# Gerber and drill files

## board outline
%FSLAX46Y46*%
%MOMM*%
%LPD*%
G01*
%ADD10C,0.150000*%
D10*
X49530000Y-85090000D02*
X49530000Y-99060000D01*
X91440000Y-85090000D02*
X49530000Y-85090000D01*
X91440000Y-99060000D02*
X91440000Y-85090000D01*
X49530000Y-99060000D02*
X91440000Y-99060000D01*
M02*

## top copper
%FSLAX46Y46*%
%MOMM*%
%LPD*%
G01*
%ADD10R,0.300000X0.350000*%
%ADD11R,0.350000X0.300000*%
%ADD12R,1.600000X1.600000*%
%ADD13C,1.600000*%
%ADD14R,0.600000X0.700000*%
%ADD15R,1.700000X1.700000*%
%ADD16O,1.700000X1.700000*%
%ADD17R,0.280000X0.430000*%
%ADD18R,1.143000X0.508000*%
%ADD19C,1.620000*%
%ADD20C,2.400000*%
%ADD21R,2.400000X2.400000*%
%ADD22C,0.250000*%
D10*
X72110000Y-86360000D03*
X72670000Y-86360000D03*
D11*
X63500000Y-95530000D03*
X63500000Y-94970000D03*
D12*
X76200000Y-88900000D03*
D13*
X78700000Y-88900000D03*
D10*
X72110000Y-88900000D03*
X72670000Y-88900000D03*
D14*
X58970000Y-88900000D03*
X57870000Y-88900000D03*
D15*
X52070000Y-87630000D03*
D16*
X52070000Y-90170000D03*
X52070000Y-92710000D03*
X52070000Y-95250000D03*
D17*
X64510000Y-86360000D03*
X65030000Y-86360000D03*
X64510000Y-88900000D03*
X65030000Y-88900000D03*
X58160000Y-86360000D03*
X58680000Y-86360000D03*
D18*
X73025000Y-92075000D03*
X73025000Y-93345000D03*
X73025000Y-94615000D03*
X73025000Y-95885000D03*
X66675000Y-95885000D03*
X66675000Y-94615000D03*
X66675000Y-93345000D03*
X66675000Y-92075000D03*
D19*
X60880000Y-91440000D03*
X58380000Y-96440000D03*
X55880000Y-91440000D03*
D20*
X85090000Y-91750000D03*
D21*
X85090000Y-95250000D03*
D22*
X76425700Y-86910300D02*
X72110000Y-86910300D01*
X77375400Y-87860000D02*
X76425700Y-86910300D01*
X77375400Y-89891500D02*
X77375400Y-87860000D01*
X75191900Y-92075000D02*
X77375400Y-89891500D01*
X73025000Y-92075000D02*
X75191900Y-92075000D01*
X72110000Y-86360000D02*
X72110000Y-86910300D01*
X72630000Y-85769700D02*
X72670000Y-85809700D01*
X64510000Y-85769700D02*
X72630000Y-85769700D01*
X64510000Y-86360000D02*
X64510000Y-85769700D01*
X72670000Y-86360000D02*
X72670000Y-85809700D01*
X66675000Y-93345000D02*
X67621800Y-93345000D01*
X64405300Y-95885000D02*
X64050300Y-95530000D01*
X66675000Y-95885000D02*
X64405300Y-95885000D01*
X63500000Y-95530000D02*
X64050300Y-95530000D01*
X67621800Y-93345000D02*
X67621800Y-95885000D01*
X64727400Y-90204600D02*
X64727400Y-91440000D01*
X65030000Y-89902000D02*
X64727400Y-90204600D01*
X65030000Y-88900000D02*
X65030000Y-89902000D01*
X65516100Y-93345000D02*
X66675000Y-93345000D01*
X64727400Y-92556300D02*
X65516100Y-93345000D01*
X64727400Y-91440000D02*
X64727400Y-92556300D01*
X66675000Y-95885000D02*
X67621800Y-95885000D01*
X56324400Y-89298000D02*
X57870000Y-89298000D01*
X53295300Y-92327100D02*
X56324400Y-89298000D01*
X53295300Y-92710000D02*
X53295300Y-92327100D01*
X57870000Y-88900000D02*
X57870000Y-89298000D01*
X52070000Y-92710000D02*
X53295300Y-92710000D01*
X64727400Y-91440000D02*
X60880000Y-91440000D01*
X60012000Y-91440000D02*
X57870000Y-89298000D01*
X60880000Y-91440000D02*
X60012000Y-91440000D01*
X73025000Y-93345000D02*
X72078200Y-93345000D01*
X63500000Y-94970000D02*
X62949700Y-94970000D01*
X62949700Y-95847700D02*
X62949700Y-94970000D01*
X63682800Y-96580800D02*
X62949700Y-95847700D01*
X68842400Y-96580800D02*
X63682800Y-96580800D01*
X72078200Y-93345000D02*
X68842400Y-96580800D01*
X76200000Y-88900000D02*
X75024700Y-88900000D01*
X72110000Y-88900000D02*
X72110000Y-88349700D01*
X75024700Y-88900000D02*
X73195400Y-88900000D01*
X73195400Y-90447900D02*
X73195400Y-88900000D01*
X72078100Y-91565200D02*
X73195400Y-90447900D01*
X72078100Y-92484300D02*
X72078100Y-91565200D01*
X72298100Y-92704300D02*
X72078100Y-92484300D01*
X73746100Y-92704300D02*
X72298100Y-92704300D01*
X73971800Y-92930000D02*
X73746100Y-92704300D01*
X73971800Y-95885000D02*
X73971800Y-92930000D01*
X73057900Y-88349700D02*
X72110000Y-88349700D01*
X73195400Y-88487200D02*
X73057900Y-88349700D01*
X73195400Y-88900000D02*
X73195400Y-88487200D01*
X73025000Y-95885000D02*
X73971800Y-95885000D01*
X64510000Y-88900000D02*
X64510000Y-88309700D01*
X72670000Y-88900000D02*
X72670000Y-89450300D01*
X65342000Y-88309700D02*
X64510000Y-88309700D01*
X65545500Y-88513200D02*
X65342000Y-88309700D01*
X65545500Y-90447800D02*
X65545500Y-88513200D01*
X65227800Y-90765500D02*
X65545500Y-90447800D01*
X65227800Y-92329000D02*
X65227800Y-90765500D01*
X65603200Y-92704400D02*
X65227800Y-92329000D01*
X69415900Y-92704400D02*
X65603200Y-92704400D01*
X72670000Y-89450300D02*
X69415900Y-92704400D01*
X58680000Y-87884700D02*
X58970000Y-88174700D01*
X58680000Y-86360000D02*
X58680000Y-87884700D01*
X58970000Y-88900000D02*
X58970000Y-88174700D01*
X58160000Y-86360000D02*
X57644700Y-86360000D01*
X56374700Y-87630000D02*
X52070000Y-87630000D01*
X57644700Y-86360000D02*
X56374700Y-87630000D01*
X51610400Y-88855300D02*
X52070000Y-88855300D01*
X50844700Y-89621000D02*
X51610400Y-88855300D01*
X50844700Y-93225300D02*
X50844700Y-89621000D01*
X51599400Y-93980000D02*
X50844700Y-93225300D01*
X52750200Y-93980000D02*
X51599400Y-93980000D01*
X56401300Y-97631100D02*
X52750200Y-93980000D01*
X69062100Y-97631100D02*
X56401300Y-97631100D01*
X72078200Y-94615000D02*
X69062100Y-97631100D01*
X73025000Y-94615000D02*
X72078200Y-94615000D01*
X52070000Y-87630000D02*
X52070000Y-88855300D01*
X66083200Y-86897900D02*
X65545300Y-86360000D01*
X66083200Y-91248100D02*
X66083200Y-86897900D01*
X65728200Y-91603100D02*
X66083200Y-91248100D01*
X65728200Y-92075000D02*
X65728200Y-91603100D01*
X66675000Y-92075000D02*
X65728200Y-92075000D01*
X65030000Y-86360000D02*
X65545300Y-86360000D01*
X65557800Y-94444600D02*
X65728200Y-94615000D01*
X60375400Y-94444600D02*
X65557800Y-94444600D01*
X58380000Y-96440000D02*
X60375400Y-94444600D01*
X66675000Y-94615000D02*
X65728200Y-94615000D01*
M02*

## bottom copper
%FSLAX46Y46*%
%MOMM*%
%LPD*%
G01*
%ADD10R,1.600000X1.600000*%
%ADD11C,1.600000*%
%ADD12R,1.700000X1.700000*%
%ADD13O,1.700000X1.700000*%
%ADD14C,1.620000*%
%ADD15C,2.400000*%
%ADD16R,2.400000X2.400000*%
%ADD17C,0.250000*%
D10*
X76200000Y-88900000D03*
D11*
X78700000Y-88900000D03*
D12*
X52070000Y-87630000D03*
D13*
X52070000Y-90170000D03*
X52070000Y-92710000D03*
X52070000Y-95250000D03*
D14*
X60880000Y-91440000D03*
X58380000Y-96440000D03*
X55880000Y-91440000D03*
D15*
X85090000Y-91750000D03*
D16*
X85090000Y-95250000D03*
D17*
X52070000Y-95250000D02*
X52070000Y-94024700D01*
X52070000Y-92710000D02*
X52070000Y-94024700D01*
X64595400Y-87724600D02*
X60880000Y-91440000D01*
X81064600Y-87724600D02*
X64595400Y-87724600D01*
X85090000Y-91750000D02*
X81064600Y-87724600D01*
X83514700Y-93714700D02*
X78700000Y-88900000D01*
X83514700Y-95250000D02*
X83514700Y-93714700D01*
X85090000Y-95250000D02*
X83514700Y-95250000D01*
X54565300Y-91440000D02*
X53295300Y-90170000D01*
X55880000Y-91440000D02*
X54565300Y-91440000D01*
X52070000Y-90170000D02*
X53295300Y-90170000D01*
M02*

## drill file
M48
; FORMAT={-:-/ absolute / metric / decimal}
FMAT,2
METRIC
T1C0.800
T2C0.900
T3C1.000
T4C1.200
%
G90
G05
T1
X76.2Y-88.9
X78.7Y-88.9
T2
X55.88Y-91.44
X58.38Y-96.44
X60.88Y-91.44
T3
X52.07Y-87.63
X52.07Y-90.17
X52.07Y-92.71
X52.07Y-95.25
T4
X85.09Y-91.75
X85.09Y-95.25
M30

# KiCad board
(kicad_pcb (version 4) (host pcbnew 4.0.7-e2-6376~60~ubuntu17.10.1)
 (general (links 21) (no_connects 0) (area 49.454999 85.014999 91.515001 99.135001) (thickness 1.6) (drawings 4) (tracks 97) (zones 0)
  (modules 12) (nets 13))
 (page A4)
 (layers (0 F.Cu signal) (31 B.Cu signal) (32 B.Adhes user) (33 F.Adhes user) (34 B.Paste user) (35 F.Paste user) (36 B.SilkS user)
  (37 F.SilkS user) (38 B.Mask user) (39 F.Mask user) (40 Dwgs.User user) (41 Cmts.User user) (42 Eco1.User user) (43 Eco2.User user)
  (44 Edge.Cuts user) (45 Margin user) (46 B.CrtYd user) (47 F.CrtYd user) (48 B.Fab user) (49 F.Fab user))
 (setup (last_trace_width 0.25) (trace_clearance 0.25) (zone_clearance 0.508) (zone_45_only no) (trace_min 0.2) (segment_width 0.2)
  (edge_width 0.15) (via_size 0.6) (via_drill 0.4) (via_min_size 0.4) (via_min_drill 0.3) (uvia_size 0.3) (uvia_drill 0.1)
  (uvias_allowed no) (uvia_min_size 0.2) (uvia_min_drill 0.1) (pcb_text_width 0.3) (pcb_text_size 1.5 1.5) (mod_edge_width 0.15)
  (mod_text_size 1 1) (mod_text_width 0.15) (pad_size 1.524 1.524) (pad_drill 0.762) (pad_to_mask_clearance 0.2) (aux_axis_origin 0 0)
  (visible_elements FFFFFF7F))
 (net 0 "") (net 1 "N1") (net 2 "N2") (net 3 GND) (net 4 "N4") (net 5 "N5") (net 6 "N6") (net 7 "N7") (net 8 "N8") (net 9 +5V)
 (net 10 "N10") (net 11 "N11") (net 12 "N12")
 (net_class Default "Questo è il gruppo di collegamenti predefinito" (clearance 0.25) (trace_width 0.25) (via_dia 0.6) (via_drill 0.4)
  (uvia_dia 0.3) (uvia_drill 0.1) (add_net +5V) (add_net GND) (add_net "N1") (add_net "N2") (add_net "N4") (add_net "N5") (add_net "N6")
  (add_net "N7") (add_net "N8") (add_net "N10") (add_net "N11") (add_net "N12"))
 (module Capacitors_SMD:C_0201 (layer F.Cu) (at 72.39 86.36)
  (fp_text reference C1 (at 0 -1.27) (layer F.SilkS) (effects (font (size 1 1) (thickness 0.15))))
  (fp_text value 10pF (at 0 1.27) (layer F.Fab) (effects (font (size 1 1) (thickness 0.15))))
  (pad 1 smd rect (at -0.28 0) (size 0.3 0.35) (layers F.Cu F.Paste F.Mask) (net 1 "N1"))
  (pad 2 smd rect (at 0.28 0) (size 0.3 0.35) (layers F.Cu F.Paste F.Mask) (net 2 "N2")))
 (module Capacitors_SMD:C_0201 (layer F.Cu) (at 63.5 95.25 90)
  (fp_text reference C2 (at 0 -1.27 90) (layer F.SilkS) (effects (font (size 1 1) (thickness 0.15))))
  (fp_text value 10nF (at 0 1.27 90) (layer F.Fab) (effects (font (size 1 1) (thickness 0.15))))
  (pad 1 smd rect (at -0.28 0 90) (size 0.3 0.35) (layers F.Cu F.Paste F.Mask) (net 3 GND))
  (pad 2 smd rect (at 0.28 0 90) (size 0.3 0.35) (layers F.Cu F.Paste F.Mask) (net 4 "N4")))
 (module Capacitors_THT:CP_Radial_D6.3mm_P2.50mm (layer F.Cu) (at 76.2 88.9)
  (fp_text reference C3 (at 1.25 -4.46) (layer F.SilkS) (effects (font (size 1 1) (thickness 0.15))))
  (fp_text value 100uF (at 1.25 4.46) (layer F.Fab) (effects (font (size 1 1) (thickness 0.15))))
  (pad 1 thru_hole rect (at 0 0) (size 1.6 1.6) (drill 0.8) (layers *.Cu *.Mask) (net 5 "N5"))
  (pad 2 thru_hole circle (at 2.5 0) (size 1.6 1.6) (drill 0.8) (layers *.Cu *.Mask) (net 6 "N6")))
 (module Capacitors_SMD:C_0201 (layer F.Cu) (at 72.39 88.9)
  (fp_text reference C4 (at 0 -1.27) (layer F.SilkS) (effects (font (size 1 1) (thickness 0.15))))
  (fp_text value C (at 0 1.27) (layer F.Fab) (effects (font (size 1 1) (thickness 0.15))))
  (pad 1 smd rect (at -0.28 0) (size 0.3 0.35) (layers F.Cu F.Paste F.Mask) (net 5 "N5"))
  (pad 2 smd rect (at 0.28 0) (size 0.3 0.35) (layers F.Cu F.Paste F.Mask) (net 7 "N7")))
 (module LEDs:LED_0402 (layer F.Cu) (at 58.42 88.9)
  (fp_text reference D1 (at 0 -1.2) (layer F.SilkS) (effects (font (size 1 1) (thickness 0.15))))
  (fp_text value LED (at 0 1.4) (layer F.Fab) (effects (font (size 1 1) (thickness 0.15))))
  (pad 2 smd rect (at 0.55 0 180) (size 0.6 0.7) (layers F.Cu F.Paste F.Mask) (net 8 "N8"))
  (pad 1 smd rect (at -0.55 0 180) (size 0.6 0.7) (layers F.Cu F.Paste F.Mask) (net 3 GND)))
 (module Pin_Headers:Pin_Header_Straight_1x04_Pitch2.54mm (layer F.Cu) (at 52.07 87.63)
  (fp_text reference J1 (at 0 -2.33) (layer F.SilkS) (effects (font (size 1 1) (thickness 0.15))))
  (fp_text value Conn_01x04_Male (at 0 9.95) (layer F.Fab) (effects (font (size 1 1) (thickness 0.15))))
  (pad 1 thru_hole rect (at 0 0) (size 1.7 1.7) (drill 1) (layers *.Cu *.Mask) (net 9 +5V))
  (pad 2 thru_hole oval (at 0 2.54) (size 1.7 1.7) (drill 1) (layers *.Cu *.Mask) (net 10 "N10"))
  (pad 3 thru_hole oval (at 0 5.08) (size 1.7 1.7) (drill 1) (layers *.Cu *.Mask) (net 3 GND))
  (pad 4 thru_hole oval (at 0 7.62) (size 1.7 1.7) (drill 1) (layers *.Cu *.Mask) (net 3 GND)))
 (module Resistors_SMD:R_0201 (layer F.Cu) (at 64.77 86.36)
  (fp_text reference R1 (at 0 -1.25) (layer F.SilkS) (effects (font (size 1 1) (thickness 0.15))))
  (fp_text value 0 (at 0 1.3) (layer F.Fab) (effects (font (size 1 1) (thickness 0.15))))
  (pad 1 smd rect (at -0.26 0) (size 0.28 0.43) (layers F.Cu F.Paste F.Mask) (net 2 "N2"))
  (pad 2 smd rect (at 0.26 0) (size 0.28 0.43) (layers F.Cu F.Paste F.Mask) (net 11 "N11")))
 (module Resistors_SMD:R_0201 (layer F.Cu) (at 64.77 88.9)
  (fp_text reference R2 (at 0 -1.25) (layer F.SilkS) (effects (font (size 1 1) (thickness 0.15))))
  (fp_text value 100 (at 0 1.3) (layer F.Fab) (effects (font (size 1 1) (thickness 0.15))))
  (pad 1 smd rect (at -0.26 0) (size 0.28 0.43) (layers F.Cu F.Paste F.Mask) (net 7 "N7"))
  (pad 2 smd rect (at 0.26 0) (size 0.28 0.43) (layers F.Cu F.Paste F.Mask) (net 3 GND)))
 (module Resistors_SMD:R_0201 (layer F.Cu) (at 58.42 86.36)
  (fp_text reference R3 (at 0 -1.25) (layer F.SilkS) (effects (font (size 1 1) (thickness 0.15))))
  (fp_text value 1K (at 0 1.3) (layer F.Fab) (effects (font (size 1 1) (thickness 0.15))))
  (pad 1 smd rect (at -0.26 0) (size 0.28 0.43) (layers F.Cu F.Paste F.Mask) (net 9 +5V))
  (pad 2 smd rect (at 0.26 0) (size 0.28 0.43) (layers F.Cu F.Paste F.Mask) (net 8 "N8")))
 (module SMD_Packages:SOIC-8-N (layer F.Cu) (at 69.85 93.98 270)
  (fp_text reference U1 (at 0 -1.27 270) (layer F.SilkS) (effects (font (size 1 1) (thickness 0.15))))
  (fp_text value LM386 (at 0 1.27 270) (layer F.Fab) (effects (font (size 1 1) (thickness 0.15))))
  (pad 8 smd rect (at -1.905 -3.175 270) (size 0.508 1.143) (layers F.Cu F.Paste F.Mask) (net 1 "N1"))
  (pad 7 smd rect (at -0.635 -3.175 270) (size 0.508 1.143) (layers F.Cu F.Paste F.Mask) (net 4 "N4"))
  (pad 6 smd rect (at 0.635 -3.175 270) (size 0.508 1.143) (layers F.Cu F.Paste F.Mask) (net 9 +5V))
  (pad 5 smd rect (at 1.905 -3.175 270) (size 0.508 1.143) (layers F.Cu F.Paste F.Mask) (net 5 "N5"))
  (pad 4 smd rect (at 1.905 3.175 270) (size 0.508 1.143) (layers F.Cu F.Paste F.Mask) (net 3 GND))
  (pad 3 smd rect (at 0.635 3.175 270) (size 0.508 1.143) (layers F.Cu F.Paste F.Mask) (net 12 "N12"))
  (pad 2 smd rect (at -0.635 3.175 270) (size 0.508 1.143) (layers F.Cu F.Paste F.Mask) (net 3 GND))
  (pad 1 smd rect (at -1.905 3.175 270) (size 0.508 1.143) (layers F.Cu F.Paste F.Mask) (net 11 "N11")))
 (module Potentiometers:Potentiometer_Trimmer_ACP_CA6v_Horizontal (layer F.Cu) (at 55.88 91.44 270)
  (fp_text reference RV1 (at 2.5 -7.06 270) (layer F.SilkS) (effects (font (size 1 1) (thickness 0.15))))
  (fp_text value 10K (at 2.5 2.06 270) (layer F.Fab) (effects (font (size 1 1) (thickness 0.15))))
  (pad 3 thru_hole circle (at 0 -5 270) (size 1.62 1.62) (drill 0.9) (layers *.Cu *.Mask) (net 3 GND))
  (pad 2 thru_hole circle (at 5 -2.5 270) (size 1.62 1.62) (drill 0.9) (layers *.Cu *.Mask) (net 12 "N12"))
  (pad 1 thru_hole circle (at 0 0 270) (size 1.62 1.62) (drill 0.9) (layers *.Cu *.Mask) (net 10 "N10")))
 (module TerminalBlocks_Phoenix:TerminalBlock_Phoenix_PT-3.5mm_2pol (layer F.Cu) (at 85.09 95.25 90)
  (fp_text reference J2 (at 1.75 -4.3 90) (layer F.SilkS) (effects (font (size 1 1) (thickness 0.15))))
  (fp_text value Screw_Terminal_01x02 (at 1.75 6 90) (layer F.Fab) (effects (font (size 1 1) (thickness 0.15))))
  (pad 2 thru_hole circle (at 3.5 0 90) (size 2.4 2.4) (drill 1.2) (layers *.Cu *.Mask) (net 3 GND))
  (pad 1 thru_hole rect (at 0 0 90) (size 2.4 2.4) (drill 1.2) (layers *.Cu *.Mask) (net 6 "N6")))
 (gr_line (start 49.53 85.09) (end 49.53 99.06) (angle 90) (layer Edge.Cuts) (width 0.15))
 (gr_line (start 91.44 85.09) (end 49.53 85.09) (angle 90) (layer Edge.Cuts) (width 0.15))
 (gr_line (start 91.44 99.06) (end 91.44 85.09) (angle 90) (layer Edge.Cuts) (width 0.15))
 (gr_line (start 49.53 99.06) (end 91.44 99.06) (angle 90) (layer Edge.Cuts) (width 0.15))
 (segment (start 76.4257 86.9103) (end 72.11 86.9103) (width 0.25) (layer F.Cu) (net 1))
 (segment (start 77.3754 87.86) (end 76.4257 86.9103) (width 0.25) (layer F.Cu) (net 1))
 (segment (start 77.3754 89.8915) (end 77.3754 87.86) (width 0.25) (layer F.Cu) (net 1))
 (segment (start 75.1919 92.075) (end 77.3754 89.8915) (width 0.25) (layer F.Cu) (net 1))
 (segment (start 73.025 92.075) (end 75.1919 92.075) (width 0.25) (layer F.Cu) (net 1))
 (segment (start 72.11 86.36) (end 72.11 86.9103) (width 0.25) (layer F.Cu) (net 1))
 (segment (start 72.63 85.7697) (end 72.67 85.8097) (width 0.25) (layer F.Cu) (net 2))
 (segment (start 64.51 85.7697) (end 72.63 85.7697) (width 0.25) (layer F.Cu) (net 2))
 (segment (start 64.51 86.36) (end 64.51 85.7697) (width 0.25) (layer F.Cu) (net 2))
 (segment (start 72.67 86.36) (end 72.67 85.8097) (width 0.25) (layer F.Cu) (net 2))
 (segment (start 66.675 93.345) (end 67.6218 93.345) (width 0.25) (layer F.Cu) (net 3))
 (segment (start 64.4053 95.885) (end 64.0503 95.53) (width 0.25) (layer F.Cu) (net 3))
 (segment (start 66.675 95.885) (end 64.4053 95.885) (width 0.25) (layer F.Cu) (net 3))
 (segment (start 63.5 95.53) (end 64.0503 95.53) (width 0.25) (layer F.Cu) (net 3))
 (segment (start 67.6218 93.345) (end 67.6218 95.885) (width 0.25) (layer F.Cu) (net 3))
 (segment (start 52.07 95.25) (end 52.07 94.0247) (width 0.25) (layer B.Cu) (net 3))
 (segment (start 52.07 92.71) (end 52.07 94.0247) (width 0.25) (layer B.Cu) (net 3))
 (segment (start 64.7274 90.2046) (end 64.7274 91.44) (width 0.25) (layer F.Cu) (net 3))
 (segment (start 65.03 89.902) (end 64.7274 90.2046) (width 0.25) (layer F.Cu) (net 3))
 (segment (start 65.03 88.9) (end 65.03 89.902) (width 0.25) (layer F.Cu) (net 3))
 (segment (start 65.5161 93.345) (end 66.675 93.345) (width 0.25) (layer F.Cu) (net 3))
 (segment (start 64.7274 92.5563) (end 65.5161 93.345) (width 0.25) (layer F.Cu) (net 3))
 (segment (start 64.7274 91.44) (end 64.7274 92.5563) (width 0.25) (layer F.Cu) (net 3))
 (segment (start 66.675 95.885) (end 67.6218 95.885) (width 0.25) (layer F.Cu) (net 3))
 (segment (start 56.3244 89.298) (end 57.87 89.298) (width 0.25) (layer F.Cu) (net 3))
 (segment (start 53.2953 92.3271) (end 56.3244 89.298) (width 0.25) (layer F.Cu) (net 3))
 (segment (start 53.2953 92.71) (end 53.2953 92.3271) (width 0.25) (layer F.Cu) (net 3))
 (segment (start 57.87 88.9) (end 57.87 89.298) (width 0.25) (layer F.Cu) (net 3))
 (segment (start 52.07 92.71) (end 53.2953 92.71) (width 0.25) (layer F.Cu) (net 3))
 (segment (start 64.7274 91.44) (end 60.88 91.44) (width 0.25) (layer F.Cu) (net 3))
 (segment (start 60.012 91.44) (end 57.87 89.298) (width 0.25) (layer F.Cu) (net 3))
 (segment (start 60.88 91.44) (end 60.012 91.44) (width 0.25) (layer F.Cu) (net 3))
 (segment (start 64.5954 87.7246) (end 60.88 91.44) (width 0.25) (layer B.Cu) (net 3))
 (segment (start 81.0646 87.7246) (end 64.5954 87.7246) (width 0.25) (layer B.Cu) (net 3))
 (segment (start 85.09 91.75) (end 81.0646 87.7246) (width 0.25) (layer B.Cu) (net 3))
 (segment (start 73.025 93.345) (end 72.0782 93.345) (width 0.25) (layer F.Cu) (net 4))
 (segment (start 63.5 94.97) (end 62.9497 94.97) (width 0.25) (layer F.Cu) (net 4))
 (segment (start 62.9497 95.8477) (end 62.9497 94.97) (width 0.25) (layer F.Cu) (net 4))
 (segment (start 63.6828 96.5808) (end 62.9497 95.8477) (width 0.25) (layer F.Cu) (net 4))
 (segment (start 68.8424 96.5808) (end 63.6828 96.5808) (width 0.25) (layer F.Cu) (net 4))
 (segment (start 72.0782 93.345) (end 68.8424 96.5808) (width 0.25) (layer F.Cu) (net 4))
 (segment (start 76.2 88.9) (end 75.0247 88.9) (width 0.25) (layer F.Cu) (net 5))
 (segment (start 72.11 88.9) (end 72.11 88.3497) (width 0.25) (layer F.Cu) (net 5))
 (segment (start 75.0247 88.9) (end 73.1954 88.9) (width 0.25) (layer F.Cu) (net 5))
 (segment (start 73.1954 90.4479) (end 73.1954 88.9) (width 0.25) (layer F.Cu) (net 5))
 (segment (start 72.0781 91.5652) (end 73.1954 90.4479) (width 0.25) (layer F.Cu) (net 5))
 (segment (start 72.0781 92.4843) (end 72.0781 91.5652) (width 0.25) (layer F.Cu) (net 5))
 (segment (start 72.2981 92.7043) (end 72.0781 92.4843) (width 0.25) (layer F.Cu) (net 5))
 (segment (start 73.7461 92.7043) (end 72.2981 92.7043) (width 0.25) (layer F.Cu) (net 5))
 (segment (start 73.9718 92.93) (end 73.7461 92.7043) (width 0.25) (layer F.Cu) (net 5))
 (segment (start 73.9718 95.885) (end 73.9718 92.93) (width 0.25) (layer F.Cu) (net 5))
 (segment (start 73.0579 88.3497) (end 72.11 88.3497) (width 0.25) (layer F.Cu) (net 5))
 (segment (start 73.1954 88.4872) (end 73.0579 88.3497) (width 0.25) (layer F.Cu) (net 5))
 (segment (start 73.1954 88.9) (end 73.1954 88.4872) (width 0.25) (layer F.Cu) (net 5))
 (segment (start 73.025 95.885) (end 73.9718 95.885) (width 0.25) (layer F.Cu) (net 5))
 (segment (start 83.5147 93.7147) (end 78.7 88.9) (width 0.25) (layer B.Cu) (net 6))
 (segment (start 83.5147 95.25) (end 83.5147 93.7147) (width 0.25) (layer B.Cu) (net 6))
 (segment (start 85.09 95.25) (end 83.5147 95.25) (width 0.25) (layer B.Cu) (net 6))
 (segment (start 64.51 88.9) (end 64.51 88.3097) (width 0.25) (layer F.Cu) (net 7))
 (segment (start 72.67 88.9) (end 72.67 89.4503) (width 0.25) (layer F.Cu) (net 7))
 (segment (start 65.342 88.3097) (end 64.51 88.3097) (width 0.25) (layer F.Cu) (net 7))
 (segment (start 65.5455 88.5132) (end 65.342 88.3097) (width 0.25) (layer F.Cu) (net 7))
 (segment (start 65.5455 90.4478) (end 65.5455 88.5132) (width 0.25) (layer F.Cu) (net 7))
 (segment (start 65.2278 90.7655) (end 65.5455 90.4478) (width 0.25) (layer F.Cu) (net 7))
 (segment (start 65.2278 92.329) (end 65.2278 90.7655) (width 0.25) (layer F.Cu) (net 7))
 (segment (start 65.6032 92.7044) (end 65.2278 92.329) (width 0.25) (layer F.Cu) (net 7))
 (segment (start 69.4159 92.7044) (end 65.6032 92.7044) (width 0.25) (layer F.Cu) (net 7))
 (segment (start 72.67 89.4503) (end 69.4159 92.7044) (width 0.25) (layer F.Cu) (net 7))
 (segment (start 58.68 87.8847) (end 58.97 88.1747) (width 0.25) (layer F.Cu) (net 8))
 (segment (start 58.68 86.36) (end 58.68 87.8847) (width 0.25) (layer F.Cu) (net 8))
 (segment (start 58.97 88.9) (end 58.97 88.1747) (width 0.25) (layer F.Cu) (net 8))
 (segment (start 58.16 86.36) (end 57.6447 86.36) (width 0.25) (layer F.Cu) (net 9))
 (segment (start 56.3747 87.63) (end 52.07 87.63) (width 0.25) (layer F.Cu) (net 9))
 (segment (start 57.6447 86.36) (end 56.3747 87.63) (width 0.25) (layer F.Cu) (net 9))
 (segment (start 51.6104 88.8553) (end 52.07 88.8553) (width 0.25) (layer F.Cu) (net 9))
 (segment (start 50.8447 89.621) (end 51.6104 88.8553) (width 0.25) (layer F.Cu) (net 9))
 (segment (start 50.8447 93.2253) (end 50.8447 89.621) (width 0.25) (layer F.Cu) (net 9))
 (segment (start 51.5994 93.98) (end 50.8447 93.2253) (width 0.25) (layer F.Cu) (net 9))
 (segment (start 52.7502 93.98) (end 51.5994 93.98) (width 0.25) (layer F.Cu) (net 9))
 (segment (start 56.4013 97.6311) (end 52.7502 93.98) (width 0.25) (layer F.Cu) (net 9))
 (segment (start 69.0621 97.6311) (end 56.4013 97.6311) (width 0.25) (layer F.Cu) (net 9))
 (segment (start 72.0782 94.615) (end 69.0621 97.6311) (width 0.25) (layer F.Cu) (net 9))
 (segment (start 73.025 94.615) (end 72.0782 94.615) (width 0.25) (layer F.Cu) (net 9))
 (segment (start 52.07 87.63) (end 52.07 88.8553) (width 0.25) (layer F.Cu) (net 9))
 (segment (start 54.5653 91.44) (end 53.2953 90.17) (width 0.25) (layer B.Cu) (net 10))
 (segment (start 55.88 91.44) (end 54.5653 91.44) (width 0.25) (layer B.Cu) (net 10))
 (segment (start 52.07 90.17) (end 53.2953 90.17) (width 0.25) (layer B.Cu) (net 10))
 (segment (start 66.0832 86.8979) (end 65.5453 86.36) (width 0.25) (layer F.Cu) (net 11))
 (segment (start 66.0832 91.2481) (end 66.0832 86.8979) (width 0.25) (layer F.Cu) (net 11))
 (segment (start 65.7282 91.6031) (end 66.0832 91.2481) (width 0.25) (layer F.Cu) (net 11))
 (segment (start 65.7282 92.075) (end 65.7282 91.6031) (width 0.25) (layer F.Cu) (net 11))
 (segment (start 66.675 92.075) (end 65.7282 92.075) (width 0.25) (layer F.Cu) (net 11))
 (segment (start 65.03 86.36) (end 65.5453 86.36) (width 0.25) (layer F.Cu) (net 11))
 (segment (start 65.5578 94.4446) (end 65.7282 94.615) (width 0.25) (layer F.Cu) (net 12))
 (segment (start 60.3754 94.4446) (end 65.5578 94.4446) (width 0.25) (layer F.Cu) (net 12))
 (segment (start 58.38 96.44) (end 60.3754 94.4446) (width 0.25) (layer F.Cu) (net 12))
 (segment (start 66.675 94.615) (end 65.7282 94.615) (width 0.25) (layer F.Cu) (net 12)))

